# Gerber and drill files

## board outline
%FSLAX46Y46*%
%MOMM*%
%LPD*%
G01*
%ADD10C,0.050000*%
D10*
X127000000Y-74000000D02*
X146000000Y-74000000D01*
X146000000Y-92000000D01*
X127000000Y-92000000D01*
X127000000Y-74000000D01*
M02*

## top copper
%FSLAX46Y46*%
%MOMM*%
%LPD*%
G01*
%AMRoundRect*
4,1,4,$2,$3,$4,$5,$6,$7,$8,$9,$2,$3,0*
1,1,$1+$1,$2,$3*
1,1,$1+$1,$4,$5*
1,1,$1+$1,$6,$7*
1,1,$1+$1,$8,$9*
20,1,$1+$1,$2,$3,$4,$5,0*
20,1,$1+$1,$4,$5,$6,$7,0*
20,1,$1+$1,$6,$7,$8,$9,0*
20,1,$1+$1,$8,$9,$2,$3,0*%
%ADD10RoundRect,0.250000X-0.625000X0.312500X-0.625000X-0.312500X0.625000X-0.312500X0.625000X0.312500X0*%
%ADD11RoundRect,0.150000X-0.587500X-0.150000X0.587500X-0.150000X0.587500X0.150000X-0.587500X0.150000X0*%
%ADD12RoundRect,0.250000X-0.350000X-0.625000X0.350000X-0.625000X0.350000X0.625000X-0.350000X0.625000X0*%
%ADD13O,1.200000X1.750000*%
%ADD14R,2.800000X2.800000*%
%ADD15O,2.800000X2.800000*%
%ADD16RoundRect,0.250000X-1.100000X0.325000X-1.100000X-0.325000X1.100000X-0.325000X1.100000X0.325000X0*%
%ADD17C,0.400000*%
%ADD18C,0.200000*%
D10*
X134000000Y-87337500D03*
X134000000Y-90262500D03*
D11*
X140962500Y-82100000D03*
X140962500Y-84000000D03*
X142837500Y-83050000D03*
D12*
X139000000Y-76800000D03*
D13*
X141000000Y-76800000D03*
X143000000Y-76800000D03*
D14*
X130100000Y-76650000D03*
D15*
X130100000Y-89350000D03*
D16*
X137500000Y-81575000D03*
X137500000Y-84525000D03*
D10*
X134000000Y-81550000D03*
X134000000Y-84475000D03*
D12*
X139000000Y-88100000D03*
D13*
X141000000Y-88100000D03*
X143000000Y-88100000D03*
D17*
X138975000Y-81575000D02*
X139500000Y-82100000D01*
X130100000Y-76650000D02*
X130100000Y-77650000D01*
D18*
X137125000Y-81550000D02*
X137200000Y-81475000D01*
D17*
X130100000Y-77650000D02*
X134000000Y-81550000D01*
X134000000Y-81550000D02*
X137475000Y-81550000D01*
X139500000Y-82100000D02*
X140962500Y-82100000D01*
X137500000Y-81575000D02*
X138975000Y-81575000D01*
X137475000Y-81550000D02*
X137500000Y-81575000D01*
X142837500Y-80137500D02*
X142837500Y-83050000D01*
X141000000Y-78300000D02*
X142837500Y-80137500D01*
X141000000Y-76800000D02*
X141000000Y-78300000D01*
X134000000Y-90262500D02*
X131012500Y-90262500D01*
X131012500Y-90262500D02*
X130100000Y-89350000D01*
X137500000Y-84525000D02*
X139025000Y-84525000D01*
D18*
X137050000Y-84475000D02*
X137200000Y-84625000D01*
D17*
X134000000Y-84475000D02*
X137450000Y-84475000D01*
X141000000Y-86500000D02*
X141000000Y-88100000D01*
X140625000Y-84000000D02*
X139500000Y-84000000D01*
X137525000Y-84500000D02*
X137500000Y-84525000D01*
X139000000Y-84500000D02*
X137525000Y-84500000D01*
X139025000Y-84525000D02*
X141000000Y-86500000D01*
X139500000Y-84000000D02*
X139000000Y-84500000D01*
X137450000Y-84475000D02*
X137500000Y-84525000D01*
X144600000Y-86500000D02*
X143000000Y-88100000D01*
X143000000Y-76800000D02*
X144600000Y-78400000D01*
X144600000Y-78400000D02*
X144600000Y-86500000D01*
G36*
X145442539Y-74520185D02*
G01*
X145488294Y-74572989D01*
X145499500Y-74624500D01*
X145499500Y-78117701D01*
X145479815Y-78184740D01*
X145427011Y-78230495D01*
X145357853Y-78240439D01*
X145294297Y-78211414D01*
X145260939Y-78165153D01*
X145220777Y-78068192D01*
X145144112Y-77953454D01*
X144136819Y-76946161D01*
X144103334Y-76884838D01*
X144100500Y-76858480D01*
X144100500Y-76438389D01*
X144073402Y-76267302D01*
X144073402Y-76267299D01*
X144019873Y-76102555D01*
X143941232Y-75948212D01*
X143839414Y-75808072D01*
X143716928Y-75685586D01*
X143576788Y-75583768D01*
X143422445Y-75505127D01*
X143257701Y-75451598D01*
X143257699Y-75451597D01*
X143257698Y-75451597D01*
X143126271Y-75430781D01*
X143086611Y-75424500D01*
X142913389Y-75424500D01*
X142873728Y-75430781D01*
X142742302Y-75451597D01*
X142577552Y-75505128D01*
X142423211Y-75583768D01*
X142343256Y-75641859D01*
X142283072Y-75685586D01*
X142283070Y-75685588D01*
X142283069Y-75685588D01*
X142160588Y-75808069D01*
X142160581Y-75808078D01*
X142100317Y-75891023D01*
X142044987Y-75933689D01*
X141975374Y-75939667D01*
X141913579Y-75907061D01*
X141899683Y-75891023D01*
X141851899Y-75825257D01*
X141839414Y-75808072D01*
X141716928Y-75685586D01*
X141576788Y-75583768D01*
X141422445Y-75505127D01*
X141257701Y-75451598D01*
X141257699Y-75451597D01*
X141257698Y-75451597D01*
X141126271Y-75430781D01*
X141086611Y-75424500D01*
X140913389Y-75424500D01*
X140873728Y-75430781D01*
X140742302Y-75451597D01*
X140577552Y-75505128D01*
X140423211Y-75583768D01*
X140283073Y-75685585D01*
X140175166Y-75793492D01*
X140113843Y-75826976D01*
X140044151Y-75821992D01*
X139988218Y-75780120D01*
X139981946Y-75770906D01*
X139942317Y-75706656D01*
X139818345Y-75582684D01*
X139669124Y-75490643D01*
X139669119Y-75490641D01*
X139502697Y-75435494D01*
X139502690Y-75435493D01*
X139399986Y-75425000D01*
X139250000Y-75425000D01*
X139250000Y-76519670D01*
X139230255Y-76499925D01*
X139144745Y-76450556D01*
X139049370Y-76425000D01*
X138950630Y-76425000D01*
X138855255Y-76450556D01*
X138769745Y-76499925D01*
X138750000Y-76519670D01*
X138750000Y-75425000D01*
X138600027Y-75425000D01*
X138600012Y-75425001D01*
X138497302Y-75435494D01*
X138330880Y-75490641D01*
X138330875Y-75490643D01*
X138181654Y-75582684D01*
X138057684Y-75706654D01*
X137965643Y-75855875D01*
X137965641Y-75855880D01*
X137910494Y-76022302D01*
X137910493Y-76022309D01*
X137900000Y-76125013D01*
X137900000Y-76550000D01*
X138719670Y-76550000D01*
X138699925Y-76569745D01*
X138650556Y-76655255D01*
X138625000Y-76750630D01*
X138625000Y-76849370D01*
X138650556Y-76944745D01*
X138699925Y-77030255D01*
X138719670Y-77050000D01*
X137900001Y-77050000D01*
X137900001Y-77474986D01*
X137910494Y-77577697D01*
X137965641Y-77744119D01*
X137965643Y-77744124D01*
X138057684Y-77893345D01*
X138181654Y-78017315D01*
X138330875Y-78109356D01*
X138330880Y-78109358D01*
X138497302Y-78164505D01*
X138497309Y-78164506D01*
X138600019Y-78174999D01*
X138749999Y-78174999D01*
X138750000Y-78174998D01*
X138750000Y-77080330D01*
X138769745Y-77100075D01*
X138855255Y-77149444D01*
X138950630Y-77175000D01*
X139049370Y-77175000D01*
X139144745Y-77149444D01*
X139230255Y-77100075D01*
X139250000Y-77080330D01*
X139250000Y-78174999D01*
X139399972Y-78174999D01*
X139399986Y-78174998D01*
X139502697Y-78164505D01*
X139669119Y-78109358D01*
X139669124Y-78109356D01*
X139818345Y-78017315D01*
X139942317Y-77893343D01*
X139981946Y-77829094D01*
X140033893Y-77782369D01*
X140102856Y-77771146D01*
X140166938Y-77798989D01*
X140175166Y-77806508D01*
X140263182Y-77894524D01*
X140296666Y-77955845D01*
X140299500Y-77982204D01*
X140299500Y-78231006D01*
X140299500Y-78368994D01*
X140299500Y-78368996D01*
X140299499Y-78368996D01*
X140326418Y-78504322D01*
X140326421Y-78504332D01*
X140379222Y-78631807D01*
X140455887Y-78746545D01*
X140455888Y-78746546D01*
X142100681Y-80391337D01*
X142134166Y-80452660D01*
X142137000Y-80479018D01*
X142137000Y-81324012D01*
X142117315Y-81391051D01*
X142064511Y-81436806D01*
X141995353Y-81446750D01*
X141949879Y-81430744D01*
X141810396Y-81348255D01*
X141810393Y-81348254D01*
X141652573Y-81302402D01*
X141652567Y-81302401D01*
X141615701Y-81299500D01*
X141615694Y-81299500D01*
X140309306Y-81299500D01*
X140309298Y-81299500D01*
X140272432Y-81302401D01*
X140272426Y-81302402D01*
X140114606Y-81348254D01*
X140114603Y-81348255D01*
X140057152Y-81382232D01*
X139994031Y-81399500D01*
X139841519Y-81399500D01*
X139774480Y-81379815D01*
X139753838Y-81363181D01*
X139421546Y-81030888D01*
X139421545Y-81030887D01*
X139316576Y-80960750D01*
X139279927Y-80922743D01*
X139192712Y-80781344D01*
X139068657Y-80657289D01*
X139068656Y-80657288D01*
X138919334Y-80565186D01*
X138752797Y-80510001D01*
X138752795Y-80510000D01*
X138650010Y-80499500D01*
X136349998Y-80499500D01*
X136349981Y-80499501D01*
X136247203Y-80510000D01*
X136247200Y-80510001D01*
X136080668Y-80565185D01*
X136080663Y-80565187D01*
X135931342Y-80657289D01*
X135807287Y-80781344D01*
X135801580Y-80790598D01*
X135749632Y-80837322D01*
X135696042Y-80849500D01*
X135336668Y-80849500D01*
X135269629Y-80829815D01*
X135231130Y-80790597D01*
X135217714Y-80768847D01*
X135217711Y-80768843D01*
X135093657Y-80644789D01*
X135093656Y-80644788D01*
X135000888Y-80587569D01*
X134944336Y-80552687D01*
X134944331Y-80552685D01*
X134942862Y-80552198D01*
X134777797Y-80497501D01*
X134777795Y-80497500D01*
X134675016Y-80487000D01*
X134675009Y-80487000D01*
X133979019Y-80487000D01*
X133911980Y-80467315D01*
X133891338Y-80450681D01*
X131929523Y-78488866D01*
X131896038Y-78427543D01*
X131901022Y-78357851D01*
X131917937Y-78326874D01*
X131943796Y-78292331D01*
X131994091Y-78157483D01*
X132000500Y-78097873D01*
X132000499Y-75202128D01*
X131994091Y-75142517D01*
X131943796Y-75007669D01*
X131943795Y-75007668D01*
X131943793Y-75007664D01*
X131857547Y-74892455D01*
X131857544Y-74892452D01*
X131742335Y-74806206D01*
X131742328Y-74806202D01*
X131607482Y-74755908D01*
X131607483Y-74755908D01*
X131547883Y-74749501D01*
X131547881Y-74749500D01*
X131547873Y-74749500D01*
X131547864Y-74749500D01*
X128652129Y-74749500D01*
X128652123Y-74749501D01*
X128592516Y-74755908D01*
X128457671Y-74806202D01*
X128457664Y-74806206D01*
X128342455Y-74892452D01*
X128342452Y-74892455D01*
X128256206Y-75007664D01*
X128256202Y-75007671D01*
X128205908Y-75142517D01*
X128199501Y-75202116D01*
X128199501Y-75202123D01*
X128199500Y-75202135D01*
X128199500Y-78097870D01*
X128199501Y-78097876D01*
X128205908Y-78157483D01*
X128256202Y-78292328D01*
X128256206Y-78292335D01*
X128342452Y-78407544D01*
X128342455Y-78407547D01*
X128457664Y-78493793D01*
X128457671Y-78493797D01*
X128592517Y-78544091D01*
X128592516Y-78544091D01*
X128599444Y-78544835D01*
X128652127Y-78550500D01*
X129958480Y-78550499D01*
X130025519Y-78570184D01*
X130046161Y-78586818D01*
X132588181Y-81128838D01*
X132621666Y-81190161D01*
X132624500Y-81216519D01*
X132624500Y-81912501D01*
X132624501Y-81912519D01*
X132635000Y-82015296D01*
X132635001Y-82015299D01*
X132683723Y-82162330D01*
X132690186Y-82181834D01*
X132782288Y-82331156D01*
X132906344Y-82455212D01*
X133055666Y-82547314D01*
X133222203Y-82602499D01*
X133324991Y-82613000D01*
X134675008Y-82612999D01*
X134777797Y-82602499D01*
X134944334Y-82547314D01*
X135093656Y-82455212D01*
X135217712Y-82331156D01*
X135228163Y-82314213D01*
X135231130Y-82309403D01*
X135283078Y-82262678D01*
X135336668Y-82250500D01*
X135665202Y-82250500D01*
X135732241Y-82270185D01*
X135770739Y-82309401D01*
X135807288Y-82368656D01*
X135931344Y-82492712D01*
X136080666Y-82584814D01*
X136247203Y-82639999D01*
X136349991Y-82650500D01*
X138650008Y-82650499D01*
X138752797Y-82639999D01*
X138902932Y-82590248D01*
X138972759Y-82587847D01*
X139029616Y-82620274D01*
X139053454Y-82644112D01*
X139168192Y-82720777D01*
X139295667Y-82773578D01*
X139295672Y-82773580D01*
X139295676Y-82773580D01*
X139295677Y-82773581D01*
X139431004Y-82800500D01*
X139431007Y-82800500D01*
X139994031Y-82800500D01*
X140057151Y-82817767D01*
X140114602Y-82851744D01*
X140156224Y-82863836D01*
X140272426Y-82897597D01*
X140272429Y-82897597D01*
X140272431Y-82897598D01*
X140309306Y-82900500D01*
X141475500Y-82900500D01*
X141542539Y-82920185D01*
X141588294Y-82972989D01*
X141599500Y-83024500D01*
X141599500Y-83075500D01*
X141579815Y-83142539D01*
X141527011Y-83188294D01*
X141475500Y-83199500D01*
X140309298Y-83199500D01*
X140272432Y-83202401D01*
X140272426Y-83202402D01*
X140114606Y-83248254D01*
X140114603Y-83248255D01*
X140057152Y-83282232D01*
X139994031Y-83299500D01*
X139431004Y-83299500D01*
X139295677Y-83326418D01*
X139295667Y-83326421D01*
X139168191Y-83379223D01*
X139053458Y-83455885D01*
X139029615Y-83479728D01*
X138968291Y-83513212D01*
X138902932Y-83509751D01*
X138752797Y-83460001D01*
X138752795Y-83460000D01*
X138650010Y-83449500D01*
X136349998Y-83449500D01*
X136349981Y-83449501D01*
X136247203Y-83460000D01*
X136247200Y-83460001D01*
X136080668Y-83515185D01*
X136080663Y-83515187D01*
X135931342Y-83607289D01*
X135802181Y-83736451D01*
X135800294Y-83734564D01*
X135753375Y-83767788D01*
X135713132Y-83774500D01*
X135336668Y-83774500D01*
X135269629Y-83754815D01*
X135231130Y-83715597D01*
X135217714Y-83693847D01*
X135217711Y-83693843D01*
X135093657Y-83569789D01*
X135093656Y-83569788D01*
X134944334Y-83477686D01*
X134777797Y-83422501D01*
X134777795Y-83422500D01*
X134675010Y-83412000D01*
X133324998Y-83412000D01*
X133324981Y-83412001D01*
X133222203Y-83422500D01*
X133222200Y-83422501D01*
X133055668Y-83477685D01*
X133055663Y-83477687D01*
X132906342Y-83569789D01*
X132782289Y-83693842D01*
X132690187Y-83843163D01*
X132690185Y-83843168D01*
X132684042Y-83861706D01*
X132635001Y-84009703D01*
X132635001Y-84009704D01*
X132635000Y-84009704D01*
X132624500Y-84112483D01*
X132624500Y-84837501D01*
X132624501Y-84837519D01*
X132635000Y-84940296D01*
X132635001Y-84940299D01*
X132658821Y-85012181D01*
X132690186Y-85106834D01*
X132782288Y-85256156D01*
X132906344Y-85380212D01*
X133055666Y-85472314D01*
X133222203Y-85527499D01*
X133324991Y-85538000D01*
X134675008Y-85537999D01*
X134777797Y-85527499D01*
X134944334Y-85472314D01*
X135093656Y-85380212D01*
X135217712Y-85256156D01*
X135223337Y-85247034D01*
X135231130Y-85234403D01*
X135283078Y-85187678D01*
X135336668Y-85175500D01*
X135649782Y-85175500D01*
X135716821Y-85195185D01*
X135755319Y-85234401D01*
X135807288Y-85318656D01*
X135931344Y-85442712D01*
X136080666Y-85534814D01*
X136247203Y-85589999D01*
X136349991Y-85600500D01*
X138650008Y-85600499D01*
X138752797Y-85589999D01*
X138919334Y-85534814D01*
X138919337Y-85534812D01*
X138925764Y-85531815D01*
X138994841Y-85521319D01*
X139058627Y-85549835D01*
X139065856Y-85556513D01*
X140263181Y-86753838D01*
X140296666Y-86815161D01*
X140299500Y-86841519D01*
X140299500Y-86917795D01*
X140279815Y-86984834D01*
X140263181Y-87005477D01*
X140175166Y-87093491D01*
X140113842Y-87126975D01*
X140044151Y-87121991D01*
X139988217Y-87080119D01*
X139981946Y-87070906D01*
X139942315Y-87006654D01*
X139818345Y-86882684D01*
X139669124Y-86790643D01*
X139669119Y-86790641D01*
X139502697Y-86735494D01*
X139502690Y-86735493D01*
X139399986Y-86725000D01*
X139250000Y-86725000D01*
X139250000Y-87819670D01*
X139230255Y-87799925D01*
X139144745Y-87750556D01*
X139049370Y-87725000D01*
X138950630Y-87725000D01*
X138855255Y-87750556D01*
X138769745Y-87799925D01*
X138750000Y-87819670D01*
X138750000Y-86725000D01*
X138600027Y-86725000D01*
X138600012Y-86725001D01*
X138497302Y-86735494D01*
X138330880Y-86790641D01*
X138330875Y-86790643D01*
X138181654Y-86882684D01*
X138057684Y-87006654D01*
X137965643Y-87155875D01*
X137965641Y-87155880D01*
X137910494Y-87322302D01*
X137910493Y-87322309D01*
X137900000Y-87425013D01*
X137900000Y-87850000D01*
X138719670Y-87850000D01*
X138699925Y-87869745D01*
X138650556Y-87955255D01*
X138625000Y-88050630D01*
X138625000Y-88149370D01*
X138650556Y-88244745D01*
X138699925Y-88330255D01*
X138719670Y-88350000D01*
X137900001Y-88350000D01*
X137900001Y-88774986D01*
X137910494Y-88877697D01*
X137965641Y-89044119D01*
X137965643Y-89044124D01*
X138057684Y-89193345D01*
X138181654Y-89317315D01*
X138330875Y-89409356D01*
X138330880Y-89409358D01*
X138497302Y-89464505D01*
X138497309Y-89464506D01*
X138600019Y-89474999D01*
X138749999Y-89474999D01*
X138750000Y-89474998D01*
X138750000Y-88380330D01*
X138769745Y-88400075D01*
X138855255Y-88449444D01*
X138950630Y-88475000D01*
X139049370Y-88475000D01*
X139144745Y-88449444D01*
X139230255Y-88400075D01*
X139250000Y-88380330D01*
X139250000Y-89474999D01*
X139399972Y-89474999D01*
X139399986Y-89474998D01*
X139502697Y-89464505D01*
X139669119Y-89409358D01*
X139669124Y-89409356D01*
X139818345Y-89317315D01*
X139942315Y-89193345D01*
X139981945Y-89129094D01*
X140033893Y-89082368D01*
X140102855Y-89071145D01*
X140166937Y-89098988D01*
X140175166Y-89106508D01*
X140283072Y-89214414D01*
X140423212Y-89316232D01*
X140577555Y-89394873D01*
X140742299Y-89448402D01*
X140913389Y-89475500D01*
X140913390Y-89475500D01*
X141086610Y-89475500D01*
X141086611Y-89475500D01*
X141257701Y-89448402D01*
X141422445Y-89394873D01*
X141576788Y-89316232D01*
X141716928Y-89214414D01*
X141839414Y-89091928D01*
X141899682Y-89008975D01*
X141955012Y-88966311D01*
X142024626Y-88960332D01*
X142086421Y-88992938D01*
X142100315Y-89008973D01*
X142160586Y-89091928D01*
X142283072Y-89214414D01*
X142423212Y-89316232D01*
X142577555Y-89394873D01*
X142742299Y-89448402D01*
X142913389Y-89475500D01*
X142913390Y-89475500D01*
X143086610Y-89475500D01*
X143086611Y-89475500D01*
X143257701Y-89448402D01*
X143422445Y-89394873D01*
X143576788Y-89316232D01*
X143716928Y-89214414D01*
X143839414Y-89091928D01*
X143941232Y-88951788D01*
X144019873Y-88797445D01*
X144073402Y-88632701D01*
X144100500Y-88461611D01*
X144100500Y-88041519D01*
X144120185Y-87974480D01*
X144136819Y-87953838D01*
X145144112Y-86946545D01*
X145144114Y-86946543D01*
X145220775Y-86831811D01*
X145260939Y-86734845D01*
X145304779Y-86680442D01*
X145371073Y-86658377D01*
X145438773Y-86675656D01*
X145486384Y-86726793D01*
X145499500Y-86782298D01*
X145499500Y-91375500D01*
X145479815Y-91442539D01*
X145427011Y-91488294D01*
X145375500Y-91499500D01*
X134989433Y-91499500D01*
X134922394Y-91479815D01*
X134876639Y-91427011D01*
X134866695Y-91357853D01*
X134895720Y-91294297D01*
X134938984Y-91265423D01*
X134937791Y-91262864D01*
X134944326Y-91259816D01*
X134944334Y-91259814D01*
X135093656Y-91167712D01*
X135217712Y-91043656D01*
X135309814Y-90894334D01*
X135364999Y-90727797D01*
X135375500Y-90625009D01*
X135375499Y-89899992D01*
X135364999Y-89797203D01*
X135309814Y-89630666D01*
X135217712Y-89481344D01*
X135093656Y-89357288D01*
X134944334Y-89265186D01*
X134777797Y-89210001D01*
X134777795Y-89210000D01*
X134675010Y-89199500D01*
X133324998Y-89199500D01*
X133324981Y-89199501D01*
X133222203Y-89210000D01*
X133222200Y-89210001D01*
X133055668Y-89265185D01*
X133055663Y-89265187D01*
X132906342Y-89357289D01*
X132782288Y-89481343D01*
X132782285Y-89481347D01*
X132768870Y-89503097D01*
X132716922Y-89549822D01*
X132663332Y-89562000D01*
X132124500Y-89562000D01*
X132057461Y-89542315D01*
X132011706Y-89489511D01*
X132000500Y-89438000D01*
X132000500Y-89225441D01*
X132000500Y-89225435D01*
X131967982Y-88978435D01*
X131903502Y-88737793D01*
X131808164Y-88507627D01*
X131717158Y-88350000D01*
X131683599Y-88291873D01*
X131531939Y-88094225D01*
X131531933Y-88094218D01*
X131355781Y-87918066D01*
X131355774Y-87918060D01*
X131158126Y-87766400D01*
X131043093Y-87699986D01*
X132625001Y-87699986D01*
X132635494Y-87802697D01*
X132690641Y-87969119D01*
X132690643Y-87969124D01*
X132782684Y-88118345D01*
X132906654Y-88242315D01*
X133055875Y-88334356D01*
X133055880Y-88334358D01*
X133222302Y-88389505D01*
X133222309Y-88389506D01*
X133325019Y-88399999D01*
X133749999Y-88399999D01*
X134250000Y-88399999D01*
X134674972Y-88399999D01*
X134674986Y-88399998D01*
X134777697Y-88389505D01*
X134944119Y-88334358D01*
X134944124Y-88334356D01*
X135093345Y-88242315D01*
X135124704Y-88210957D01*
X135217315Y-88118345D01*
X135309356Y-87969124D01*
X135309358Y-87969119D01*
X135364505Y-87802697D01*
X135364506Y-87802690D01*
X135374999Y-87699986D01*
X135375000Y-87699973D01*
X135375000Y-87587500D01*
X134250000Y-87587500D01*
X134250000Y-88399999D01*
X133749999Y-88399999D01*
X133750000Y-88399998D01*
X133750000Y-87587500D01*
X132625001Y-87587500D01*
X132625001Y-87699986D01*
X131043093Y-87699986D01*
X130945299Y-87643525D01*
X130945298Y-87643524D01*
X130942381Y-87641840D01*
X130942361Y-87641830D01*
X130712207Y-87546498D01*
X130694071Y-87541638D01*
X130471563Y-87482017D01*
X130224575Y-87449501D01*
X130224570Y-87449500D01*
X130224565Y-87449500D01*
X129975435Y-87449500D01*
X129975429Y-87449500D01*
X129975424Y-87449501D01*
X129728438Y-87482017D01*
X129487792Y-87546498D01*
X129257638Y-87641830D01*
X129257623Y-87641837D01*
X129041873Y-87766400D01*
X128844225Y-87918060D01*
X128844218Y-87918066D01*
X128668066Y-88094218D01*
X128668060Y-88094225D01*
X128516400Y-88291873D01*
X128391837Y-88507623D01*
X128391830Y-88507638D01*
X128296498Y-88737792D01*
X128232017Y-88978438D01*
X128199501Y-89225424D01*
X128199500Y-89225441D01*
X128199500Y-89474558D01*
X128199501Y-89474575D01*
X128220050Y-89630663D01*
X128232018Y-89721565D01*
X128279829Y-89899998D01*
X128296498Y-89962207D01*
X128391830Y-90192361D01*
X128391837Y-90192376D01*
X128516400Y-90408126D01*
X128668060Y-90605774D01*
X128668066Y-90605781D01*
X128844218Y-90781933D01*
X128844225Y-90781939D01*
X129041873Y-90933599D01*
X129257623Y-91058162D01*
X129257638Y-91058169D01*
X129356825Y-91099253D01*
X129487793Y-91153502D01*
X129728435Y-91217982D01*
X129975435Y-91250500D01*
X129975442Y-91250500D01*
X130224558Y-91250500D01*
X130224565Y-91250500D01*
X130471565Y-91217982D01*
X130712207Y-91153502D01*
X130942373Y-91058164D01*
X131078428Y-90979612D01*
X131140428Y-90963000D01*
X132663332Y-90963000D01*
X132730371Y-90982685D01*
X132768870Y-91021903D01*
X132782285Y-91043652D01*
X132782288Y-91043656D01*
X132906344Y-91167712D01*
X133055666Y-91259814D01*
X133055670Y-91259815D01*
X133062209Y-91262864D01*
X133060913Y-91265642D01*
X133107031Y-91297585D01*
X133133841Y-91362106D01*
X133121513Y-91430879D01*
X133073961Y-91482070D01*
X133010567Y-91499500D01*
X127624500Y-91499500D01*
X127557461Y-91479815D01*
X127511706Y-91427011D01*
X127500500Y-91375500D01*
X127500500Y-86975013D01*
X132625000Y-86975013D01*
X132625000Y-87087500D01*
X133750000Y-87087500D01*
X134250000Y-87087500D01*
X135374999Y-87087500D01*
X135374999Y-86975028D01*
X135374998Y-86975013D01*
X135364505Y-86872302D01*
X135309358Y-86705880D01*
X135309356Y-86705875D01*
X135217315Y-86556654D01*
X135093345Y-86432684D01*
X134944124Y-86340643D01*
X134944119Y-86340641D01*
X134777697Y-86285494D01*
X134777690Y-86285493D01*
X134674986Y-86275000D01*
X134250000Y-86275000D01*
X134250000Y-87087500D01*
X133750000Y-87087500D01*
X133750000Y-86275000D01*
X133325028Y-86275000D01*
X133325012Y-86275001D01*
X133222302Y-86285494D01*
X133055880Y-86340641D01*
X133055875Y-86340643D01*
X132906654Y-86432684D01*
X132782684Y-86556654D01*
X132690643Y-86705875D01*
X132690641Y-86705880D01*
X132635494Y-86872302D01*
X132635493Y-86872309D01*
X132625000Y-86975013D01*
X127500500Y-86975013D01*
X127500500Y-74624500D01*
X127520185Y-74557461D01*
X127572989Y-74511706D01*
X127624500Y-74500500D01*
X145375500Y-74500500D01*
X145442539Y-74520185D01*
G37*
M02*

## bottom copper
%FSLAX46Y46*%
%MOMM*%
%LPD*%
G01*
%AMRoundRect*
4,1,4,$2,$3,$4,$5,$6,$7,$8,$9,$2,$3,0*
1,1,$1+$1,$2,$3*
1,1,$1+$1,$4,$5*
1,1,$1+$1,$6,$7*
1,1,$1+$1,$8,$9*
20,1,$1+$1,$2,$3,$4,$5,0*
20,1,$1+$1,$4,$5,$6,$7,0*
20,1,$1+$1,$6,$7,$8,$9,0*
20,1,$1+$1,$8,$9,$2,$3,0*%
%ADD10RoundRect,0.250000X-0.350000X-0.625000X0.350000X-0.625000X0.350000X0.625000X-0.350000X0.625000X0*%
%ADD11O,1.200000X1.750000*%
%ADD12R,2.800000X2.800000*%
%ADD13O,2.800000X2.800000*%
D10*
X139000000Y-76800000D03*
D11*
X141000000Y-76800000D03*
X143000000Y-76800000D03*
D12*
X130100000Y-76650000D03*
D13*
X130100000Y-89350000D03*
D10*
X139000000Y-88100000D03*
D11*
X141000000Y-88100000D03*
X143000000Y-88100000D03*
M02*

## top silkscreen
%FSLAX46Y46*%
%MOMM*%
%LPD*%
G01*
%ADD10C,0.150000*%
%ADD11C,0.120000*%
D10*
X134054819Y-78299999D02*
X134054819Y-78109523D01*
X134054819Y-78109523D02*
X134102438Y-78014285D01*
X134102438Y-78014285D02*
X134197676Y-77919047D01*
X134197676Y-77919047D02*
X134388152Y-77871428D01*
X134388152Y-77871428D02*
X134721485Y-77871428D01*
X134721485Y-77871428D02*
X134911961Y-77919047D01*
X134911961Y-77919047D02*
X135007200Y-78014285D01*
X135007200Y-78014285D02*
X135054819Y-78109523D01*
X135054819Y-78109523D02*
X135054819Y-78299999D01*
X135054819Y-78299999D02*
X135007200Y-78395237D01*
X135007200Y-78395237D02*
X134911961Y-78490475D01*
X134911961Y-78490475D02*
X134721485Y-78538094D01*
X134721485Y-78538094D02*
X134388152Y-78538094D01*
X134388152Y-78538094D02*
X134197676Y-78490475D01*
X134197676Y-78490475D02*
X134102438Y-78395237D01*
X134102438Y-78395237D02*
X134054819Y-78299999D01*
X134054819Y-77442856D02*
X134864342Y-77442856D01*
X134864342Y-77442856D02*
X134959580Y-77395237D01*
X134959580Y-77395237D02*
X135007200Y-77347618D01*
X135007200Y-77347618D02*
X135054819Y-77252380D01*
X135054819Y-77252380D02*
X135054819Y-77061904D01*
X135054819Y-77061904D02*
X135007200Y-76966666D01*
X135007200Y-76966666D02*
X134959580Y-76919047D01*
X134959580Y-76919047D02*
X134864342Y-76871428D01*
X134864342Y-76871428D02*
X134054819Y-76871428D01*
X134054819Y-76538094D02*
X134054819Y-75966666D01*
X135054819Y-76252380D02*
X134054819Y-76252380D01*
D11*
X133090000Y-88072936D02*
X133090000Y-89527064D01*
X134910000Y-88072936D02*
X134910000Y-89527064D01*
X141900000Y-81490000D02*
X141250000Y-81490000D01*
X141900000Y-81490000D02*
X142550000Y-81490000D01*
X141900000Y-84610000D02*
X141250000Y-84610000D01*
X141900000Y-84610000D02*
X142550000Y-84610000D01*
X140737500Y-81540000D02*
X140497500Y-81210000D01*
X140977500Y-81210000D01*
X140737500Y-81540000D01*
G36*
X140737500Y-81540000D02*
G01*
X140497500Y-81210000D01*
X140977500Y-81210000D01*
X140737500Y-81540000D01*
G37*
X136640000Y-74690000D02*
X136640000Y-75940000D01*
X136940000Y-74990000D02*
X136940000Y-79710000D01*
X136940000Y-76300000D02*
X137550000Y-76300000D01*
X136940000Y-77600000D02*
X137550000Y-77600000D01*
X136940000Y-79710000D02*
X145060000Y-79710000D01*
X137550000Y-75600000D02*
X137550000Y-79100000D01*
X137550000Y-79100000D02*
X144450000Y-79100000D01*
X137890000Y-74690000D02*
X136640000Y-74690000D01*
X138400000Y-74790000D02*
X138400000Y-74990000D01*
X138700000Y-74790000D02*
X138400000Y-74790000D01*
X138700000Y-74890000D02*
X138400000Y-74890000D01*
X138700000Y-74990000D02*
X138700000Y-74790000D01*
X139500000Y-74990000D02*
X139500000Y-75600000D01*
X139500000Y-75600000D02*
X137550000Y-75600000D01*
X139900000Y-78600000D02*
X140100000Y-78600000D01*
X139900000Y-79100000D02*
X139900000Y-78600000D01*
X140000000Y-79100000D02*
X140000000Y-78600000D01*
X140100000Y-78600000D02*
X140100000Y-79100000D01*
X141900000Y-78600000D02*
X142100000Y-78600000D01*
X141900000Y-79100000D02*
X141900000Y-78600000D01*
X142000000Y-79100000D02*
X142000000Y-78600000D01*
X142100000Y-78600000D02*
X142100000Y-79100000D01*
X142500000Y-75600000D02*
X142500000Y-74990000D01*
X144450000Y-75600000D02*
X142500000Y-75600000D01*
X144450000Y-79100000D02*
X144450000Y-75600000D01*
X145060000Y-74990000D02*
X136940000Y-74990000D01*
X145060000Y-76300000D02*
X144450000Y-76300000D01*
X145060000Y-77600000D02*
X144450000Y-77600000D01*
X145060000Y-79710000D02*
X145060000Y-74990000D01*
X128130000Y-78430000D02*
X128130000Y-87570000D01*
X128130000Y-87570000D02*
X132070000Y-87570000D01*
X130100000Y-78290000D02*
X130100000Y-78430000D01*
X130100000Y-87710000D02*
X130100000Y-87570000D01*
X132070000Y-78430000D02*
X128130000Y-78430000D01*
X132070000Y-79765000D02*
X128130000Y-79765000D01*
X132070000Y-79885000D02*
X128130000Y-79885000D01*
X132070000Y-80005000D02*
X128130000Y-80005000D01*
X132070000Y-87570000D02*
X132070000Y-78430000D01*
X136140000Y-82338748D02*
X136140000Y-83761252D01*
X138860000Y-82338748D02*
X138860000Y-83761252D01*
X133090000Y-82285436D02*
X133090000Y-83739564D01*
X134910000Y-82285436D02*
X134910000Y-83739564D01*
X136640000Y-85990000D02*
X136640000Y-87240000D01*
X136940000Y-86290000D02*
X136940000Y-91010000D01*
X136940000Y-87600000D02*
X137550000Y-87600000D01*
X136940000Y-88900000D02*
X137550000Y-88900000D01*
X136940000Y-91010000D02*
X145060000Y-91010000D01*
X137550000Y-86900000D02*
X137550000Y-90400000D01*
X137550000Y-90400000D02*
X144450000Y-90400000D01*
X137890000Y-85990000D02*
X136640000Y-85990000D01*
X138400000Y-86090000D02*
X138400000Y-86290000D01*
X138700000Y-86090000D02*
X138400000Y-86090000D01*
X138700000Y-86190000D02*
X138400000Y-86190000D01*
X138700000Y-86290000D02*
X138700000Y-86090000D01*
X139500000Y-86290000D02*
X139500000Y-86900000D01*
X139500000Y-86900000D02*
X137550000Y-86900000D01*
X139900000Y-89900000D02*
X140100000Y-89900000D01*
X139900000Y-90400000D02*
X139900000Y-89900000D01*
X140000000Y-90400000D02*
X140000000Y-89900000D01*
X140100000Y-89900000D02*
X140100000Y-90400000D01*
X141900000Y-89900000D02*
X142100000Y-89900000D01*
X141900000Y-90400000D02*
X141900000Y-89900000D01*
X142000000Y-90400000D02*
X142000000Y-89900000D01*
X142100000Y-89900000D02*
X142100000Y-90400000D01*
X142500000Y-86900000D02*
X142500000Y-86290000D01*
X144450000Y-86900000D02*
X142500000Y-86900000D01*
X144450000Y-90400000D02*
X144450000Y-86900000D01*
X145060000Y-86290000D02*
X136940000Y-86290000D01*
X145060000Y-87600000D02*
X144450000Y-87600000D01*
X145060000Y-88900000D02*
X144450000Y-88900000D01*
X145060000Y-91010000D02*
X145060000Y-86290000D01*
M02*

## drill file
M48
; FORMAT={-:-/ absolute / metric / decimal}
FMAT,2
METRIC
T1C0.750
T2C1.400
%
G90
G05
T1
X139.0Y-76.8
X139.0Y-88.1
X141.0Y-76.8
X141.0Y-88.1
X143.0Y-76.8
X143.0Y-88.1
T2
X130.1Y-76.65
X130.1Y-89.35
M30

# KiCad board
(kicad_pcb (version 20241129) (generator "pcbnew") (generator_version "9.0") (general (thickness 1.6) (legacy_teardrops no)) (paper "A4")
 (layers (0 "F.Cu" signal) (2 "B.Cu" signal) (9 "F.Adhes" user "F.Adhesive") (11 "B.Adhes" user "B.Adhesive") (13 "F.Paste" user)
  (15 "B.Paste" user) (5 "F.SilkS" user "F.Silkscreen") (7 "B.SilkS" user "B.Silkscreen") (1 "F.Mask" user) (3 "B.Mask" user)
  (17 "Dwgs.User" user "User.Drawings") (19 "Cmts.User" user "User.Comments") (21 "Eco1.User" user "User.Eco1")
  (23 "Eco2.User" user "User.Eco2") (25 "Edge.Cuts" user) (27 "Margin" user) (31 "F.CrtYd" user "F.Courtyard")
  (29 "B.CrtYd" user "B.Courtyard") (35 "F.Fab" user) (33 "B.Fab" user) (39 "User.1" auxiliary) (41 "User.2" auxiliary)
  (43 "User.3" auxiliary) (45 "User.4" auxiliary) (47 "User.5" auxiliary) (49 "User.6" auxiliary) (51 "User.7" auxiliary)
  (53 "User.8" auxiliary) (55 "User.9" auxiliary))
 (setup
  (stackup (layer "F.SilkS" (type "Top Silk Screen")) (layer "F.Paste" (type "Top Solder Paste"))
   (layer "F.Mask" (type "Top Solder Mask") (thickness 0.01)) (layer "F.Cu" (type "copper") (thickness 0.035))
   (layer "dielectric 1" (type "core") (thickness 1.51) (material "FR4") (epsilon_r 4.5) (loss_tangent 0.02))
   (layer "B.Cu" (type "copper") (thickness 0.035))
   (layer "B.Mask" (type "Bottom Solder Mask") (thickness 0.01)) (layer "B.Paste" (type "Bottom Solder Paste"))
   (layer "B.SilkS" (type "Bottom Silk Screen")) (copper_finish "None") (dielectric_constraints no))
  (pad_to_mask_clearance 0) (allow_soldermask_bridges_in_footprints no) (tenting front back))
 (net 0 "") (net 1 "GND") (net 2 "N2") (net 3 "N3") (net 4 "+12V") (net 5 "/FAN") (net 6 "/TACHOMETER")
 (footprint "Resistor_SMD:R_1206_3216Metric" (layer "F.Cu") (at 134 88.8 -90)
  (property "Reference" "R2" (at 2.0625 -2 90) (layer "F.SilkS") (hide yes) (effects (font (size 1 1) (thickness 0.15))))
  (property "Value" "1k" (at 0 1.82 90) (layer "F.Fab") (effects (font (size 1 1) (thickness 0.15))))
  (fp_line (start -0.727064 0.91) (end 0.727064 0.91) (stroke (width 0.12) (type solid)) (layer "F.SilkS"))
  (fp_line (start -0.727064 -0.91) (end 0.727064 -0.91) (stroke (width 0.12) (type solid)) (layer "F.SilkS"))
  (pad "1" smd roundrect (at -1.4625 0 270) (size 1.125 1.75) (layers "F.Cu" "F.Mask" "F.Paste") (roundrect_rratio 0.222222) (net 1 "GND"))
  (pad "2" smd roundrect (at 1.4625 0 270) (size 1.125 1.75) (layers "F.Cu" "F.Mask" "F.Paste") (roundrect_rratio 0.222222) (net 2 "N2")))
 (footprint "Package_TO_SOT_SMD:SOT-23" (layer "F.Cu") (at 141.9 83.05)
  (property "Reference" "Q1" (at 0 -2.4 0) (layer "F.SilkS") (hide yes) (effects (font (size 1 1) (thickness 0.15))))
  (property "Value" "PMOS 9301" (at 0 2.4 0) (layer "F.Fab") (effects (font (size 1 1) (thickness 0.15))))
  (fp_line (start 0 -1.56) (end -0.65 -1.56) (stroke (width 0.12) (type solid)) (layer "F.SilkS"))
  (fp_line (start 0 -1.56) (end 0.65 -1.56) (stroke (width 0.12) (type solid)) (layer "F.SilkS"))
  (fp_line (start 0 1.56) (end -0.65 1.56) (stroke (width 0.12) (type solid)) (layer "F.SilkS"))
  (fp_line (start 0 1.56) (end 0.65 1.56) (stroke (width 0.12) (type solid)) (layer "F.SilkS"))
  (fp_poly
   (pts (xy -1.1625 -1.51) (xy -1.4025 -1.84) (xy -0.9225 -1.84) (xy -1.1625 -1.51)) (stroke (width 0.12) (type solid)) (fill yes)
   (layer "F.SilkS"))
  (pad "1" smd roundrect (at -0.9375 -0.95) (size 1.475 0.6) (layers "F.Cu" "F.Mask" "F.Paste") (roundrect_rratio 0.25) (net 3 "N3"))
  (pad "2" smd roundrect (at -0.9375 0.95) (size 1.475 0.6) (layers "F.Cu" "F.Mask" "F.Paste") (roundrect_rratio 0.25) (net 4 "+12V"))
  (pad "3" smd roundrect (at 0.9375 0) (size 1.475 0.6) (layers "F.Cu" "F.Mask" "F.Paste") (roundrect_rratio 0.25) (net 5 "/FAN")))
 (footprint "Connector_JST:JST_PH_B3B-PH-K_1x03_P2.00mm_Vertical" (layer "F.Cu") (at 139 76.8)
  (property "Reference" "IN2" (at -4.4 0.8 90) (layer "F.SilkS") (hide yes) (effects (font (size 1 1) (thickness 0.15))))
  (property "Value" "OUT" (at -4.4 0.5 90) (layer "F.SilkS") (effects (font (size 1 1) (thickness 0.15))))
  (fp_line (start -2.36 -2.11) (end -2.36 -0.86) (stroke (width 0.12) (type solid)) (layer "F.SilkS"))
  (fp_line (start -2.06 -1.81) (end -2.06 2.91) (stroke (width 0.12) (type solid)) (layer "F.SilkS"))
  (fp_line (start -2.06 -0.5) (end -1.45 -0.5) (stroke (width 0.12) (type solid)) (layer "F.SilkS"))
  (fp_line (start -2.06 0.8) (end -1.45 0.8) (stroke (width 0.12) (type solid)) (layer "F.SilkS"))
  (fp_line (start -2.06 2.91) (end 6.06 2.91) (stroke (width 0.12) (type solid)) (layer "F.SilkS"))
  (fp_line (start -1.45 -1.2) (end -1.45 2.3) (stroke (width 0.12) (type solid)) (layer "F.SilkS"))
  (fp_line (start -1.45 2.3) (end 5.45 2.3) (stroke (width 0.12) (type solid)) (layer "F.SilkS"))
  (fp_line (start -1.11 -2.11) (end -2.36 -2.11) (stroke (width 0.12) (type solid)) (layer "F.SilkS"))
  (fp_line (start -0.6 -2.01) (end -0.6 -1.81) (stroke (width 0.12) (type solid)) (layer "F.SilkS"))
  (fp_line (start -0.3 -2.01) (end -0.6 -2.01) (stroke (width 0.12) (type solid)) (layer "F.SilkS"))
  (fp_line (start -0.3 -1.91) (end -0.6 -1.91) (stroke (width 0.12) (type solid)) (layer "F.SilkS"))
  (fp_line (start -0.3 -1.81) (end -0.3 -2.01) (stroke (width 0.12) (type solid)) (layer "F.SilkS"))
  (fp_line (start 0.5 -1.81) (end 0.5 -1.2) (stroke (width 0.12) (type solid)) (layer "F.SilkS"))
  (fp_line (start 0.5 -1.2) (end -1.45 -1.2) (stroke (width 0.12) (type solid)) (layer "F.SilkS"))
  (fp_line (start 0.9 1.8) (end 1.1 1.8) (stroke (width 0.12) (type solid)) (layer "F.SilkS"))
  (fp_line (start 0.9 2.3) (end 0.9 1.8) (stroke (width 0.12) (type solid)) (layer "F.SilkS"))
  (fp_line (start 1 2.3) (end 1 1.8) (stroke (width 0.12) (type solid)) (layer "F.SilkS"))
  (fp_line (start 1.1 1.8) (end 1.1 2.3) (stroke (width 0.12) (type solid)) (layer "F.SilkS"))
  (fp_line (start 2.9 1.8) (end 3.1 1.8) (stroke (width 0.12) (type solid)) (layer "F.SilkS"))
  (fp_line (start 2.9 2.3) (end 2.9 1.8) (stroke (width 0.12) (type solid)) (layer "F.SilkS"))
  (fp_line (start 3 2.3) (end 3 1.8) (stroke (width 0.12) (type solid)) (layer "F.SilkS"))
  (fp_line (start 3.1 1.8) (end 3.1 2.3) (stroke (width 0.12) (type solid)) (layer "F.SilkS"))
  (fp_line (start 3.5 -1.2) (end 3.5 -1.81) (stroke (width 0.12) (type solid)) (layer "F.SilkS"))
  (fp_line (start 5.45 -1.2) (end 3.5 -1.2) (stroke (width 0.12) (type solid)) (layer "F.SilkS"))
  (fp_line (start 5.45 2.3) (end 5.45 -1.2) (stroke (width 0.12) (type solid)) (layer "F.SilkS"))
  (fp_line (start 6.06 -1.81) (end -2.06 -1.81) (stroke (width 0.12) (type solid)) (layer "F.SilkS"))
  (fp_line (start 6.06 -0.5) (end 5.45 -0.5) (stroke (width 0.12) (type solid)) (layer "F.SilkS"))
  (fp_line (start 6.06 0.8) (end 5.45 0.8) (stroke (width 0.12) (type solid)) (layer "F.SilkS"))
  (fp_line (start 6.06 2.91) (end 6.06 -1.81) (stroke (width 0.12) (type solid)) (layer "F.SilkS"))
  (pad "1" thru_hole roundrect (at 0 0) (size 1.2 1.75) (drill 0.75) (layers "*.Cu" "*.Mask") (remove_unused_layers no)
   (roundrect_rratio 0.208333) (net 1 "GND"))
  (pad "2" thru_hole oval (at 2 0) (size 1.2 1.75) (drill 0.75) (layers "*.Cu" "*.Mask") (remove_unused_layers no) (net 5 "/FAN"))
  (pad "3" thru_hole oval (at 4 0) (size 1.2 1.75) (drill 0.75) (layers "*.Cu" "*.Mask") (remove_unused_layers no) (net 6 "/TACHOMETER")))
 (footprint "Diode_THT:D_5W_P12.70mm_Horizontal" (layer "F.Cu") (at 130.1 76.65 -90)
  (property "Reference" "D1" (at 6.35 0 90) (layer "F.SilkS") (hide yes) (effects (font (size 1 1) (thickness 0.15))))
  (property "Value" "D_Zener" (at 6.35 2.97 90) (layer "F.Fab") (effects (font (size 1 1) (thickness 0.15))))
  (fp_line (start 1.78 1.97) (end 10.92 1.97) (stroke (width 0.12) (type solid)) (layer "F.SilkS"))
  (fp_line (start 10.92 1.97) (end 10.92 -1.97) (stroke (width 0.12) (type solid)) (layer "F.SilkS"))
  (fp_line (start 1.64 0) (end 1.78 0) (stroke (width 0.12) (type solid)) (layer "F.SilkS"))
  (fp_line (start 11.06 0) (end 10.92 0) (stroke (width 0.12) (type solid)) (layer "F.SilkS"))
  (fp_line (start 1.78 -1.97) (end 1.78 1.97) (stroke (width 0.12) (type solid)) (layer "F.SilkS"))
  (fp_line (start 3.115 -1.97) (end 3.115 1.97) (stroke (width 0.12) (type solid)) (layer "F.SilkS"))
  (fp_line (start 3.235 -1.97) (end 3.235 1.97) (stroke (width 0.12) (type solid)) (layer "F.SilkS"))
  (fp_line (start 3.355 -1.97) (end 3.355 1.97) (stroke (width 0.12) (type solid)) (layer "F.SilkS"))
  (fp_line (start 10.92 -1.97) (end 1.78 -1.97) (stroke (width 0.12) (type solid)) (layer "F.SilkS"))
  (pad "1" thru_hole rect (at 0 0 270) (size 2.8 2.8) (drill 1.4) (layers "*.Cu" "*.Mask") (remove_unused_layers no) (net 3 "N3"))
  (pad "2" thru_hole oval (at 12.7 0 270) (size 2.8 2.8) (drill 1.4) (layers "*.Cu" "*.Mask") (remove_unused_layers no) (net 2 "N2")))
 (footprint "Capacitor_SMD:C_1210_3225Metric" (layer "F.Cu") (at 137.5 83.05 -90)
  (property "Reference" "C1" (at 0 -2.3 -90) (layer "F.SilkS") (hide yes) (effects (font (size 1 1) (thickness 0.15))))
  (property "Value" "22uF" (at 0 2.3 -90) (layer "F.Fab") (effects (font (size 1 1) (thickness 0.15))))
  (fp_line (start -0.711252 1.36) (end 0.711252 1.36) (stroke (width 0.12) (type solid)) (layer "F.SilkS"))
  (fp_line (start -0.711252 -1.36) (end 0.711252 -1.36) (stroke (width 0.12) (type solid)) (layer "F.SilkS"))
  (pad "1" smd roundrect (at -1.475 0 270) (size 1.15 2.7) (layers "F.Cu" "F.Mask" "F.Paste") (roundrect_rratio 0.217391) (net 3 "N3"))
  (pad "2" smd roundrect (at 1.475 0 270) (size 1.15 2.7) (layers "F.Cu" "F.Mask" "F.Paste") (roundrect_rratio 0.217391) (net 4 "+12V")))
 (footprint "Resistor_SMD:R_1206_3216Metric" (layer "F.Cu") (at 134 83.0125 -90)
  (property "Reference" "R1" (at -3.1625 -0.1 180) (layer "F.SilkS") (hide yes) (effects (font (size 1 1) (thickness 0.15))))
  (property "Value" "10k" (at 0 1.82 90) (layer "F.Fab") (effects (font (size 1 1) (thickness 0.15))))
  (fp_line (start -0.727064 0.91) (end 0.727064 0.91) (stroke (width 0.12) (type solid)) (layer "F.SilkS"))
  (fp_line (start -0.727064 -0.91) (end 0.727064 -0.91) (stroke (width 0.12) (type solid)) (layer "F.SilkS"))
  (pad "1" smd roundrect (at -1.4625 0 270) (size 1.125 1.75) (layers "F.Cu" "F.Mask" "F.Paste") (roundrect_rratio 0.222222) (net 3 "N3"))
  (pad "2" smd roundrect (at 1.4625 0 270) (size 1.125 1.75) (layers "F.Cu" "F.Mask" "F.Paste") (roundrect_rratio 0.222222) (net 4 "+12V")))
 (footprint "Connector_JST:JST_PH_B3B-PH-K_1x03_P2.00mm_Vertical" (layer "F.Cu") (at 139 88.1)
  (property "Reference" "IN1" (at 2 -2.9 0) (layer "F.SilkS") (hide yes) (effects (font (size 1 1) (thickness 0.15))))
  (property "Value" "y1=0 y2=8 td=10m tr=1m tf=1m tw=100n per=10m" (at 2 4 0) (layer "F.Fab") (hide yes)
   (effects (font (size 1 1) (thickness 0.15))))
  (fp_line (start -2.36 -2.11) (end -2.36 -0.86) (stroke (width 0.12) (type solid)) (layer "F.SilkS"))
  (fp_line (start -2.06 -1.81) (end -2.06 2.91) (stroke (width 0.12) (type solid)) (layer "F.SilkS"))
  (fp_line (start -2.06 -0.5) (end -1.45 -0.5) (stroke (width 0.12) (type solid)) (layer "F.SilkS"))
  (fp_line (start -2.06 0.8) (end -1.45 0.8) (stroke (width 0.12) (type solid)) (layer "F.SilkS"))
  (fp_line (start -2.06 2.91) (end 6.06 2.91) (stroke (width 0.12) (type solid)) (layer "F.SilkS"))
  (fp_line (start -1.45 -1.2) (end -1.45 2.3) (stroke (width 0.12) (type solid)) (layer "F.SilkS"))
  (fp_line (start -1.45 2.3) (end 5.45 2.3) (stroke (width 0.12) (type solid)) (layer "F.SilkS"))
  (fp_line (start -1.11 -2.11) (end -2.36 -2.11) (stroke (width 0.12) (type solid)) (layer "F.SilkS"))
  (fp_line (start -0.6 -2.01) (end -0.6 -1.81) (stroke (width 0.12) (type solid)) (layer "F.SilkS"))
  (fp_line (start -0.3 -2.01) (end -0.6 -2.01) (stroke (width 0.12) (type solid)) (layer "F.SilkS"))
  (fp_line (start -0.3 -1.91) (end -0.6 -1.91) (stroke (width 0.12) (type solid)) (layer "F.SilkS"))
  (fp_line (start -0.3 -1.81) (end -0.3 -2.01) (stroke (width 0.12) (type solid)) (layer "F.SilkS"))
  (fp_line (start 0.5 -1.81) (end 0.5 -1.2) (stroke (width 0.12) (type solid)) (layer "F.SilkS"))
  (fp_line (start 0.5 -1.2) (end -1.45 -1.2) (stroke (width 0.12) (type solid)) (layer "F.SilkS"))
  (fp_line (start 0.9 1.8) (end 1.1 1.8) (stroke (width 0.12) (type solid)) (layer "F.SilkS"))
  (fp_line (start 0.9 2.3) (end 0.9 1.8) (stroke (width 0.12) (type solid)) (layer "F.SilkS"))
  (fp_line (start 1 2.3) (end 1 1.8) (stroke (width 0.12) (type solid)) (layer "F.SilkS"))
  (fp_line (start 1.1 1.8) (end 1.1 2.3) (stroke (width 0.12) (type solid)) (layer "F.SilkS"))
  (fp_line (start 2.9 1.8) (end 3.1 1.8) (stroke (width 0.12) (type solid)) (layer "F.SilkS"))
  (fp_line (start 2.9 2.3) (end 2.9 1.8) (stroke (width 0.12) (type solid)) (layer "F.SilkS"))
  (fp_line (start 3 2.3) (end 3 1.8) (stroke (width 0.12) (type solid)) (layer "F.SilkS"))
  (fp_line (start 3.1 1.8) (end 3.1 2.3) (stroke (width 0.12) (type solid)) (layer "F.SilkS"))
  (fp_line (start 3.5 -1.2) (end 3.5 -1.81) (stroke (width 0.12) (type solid)) (layer "F.SilkS"))
  (fp_line (start 5.45 -1.2) (end 3.5 -1.2) (stroke (width 0.12) (type solid)) (layer "F.SilkS"))
  (fp_line (start 5.45 2.3) (end 5.45 -1.2) (stroke (width 0.12) (type solid)) (layer "F.SilkS"))
  (fp_line (start 6.06 -1.81) (end -2.06 -1.81) (stroke (width 0.12) (type solid)) (layer "F.SilkS"))
  (fp_line (start 6.06 -0.5) (end 5.45 -0.5) (stroke (width 0.12) (type solid)) (layer "F.SilkS"))
  (fp_line (start 6.06 0.8) (end 5.45 0.8) (stroke (width 0.12) (type solid)) (layer "F.SilkS"))
  (fp_line (start 6.06 2.91) (end 6.06 -1.81) (stroke (width 0.12) (type solid)) (layer "F.SilkS"))
  (pad "1" thru_hole roundrect (at 0 0) (size 1.2 1.75) (drill 0.75) (layers "*.Cu" "*.Mask") (remove_unused_layers no)
   (roundrect_rratio 0.208333) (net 1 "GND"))
  (pad "2" thru_hole oval (at 2 0) (size 1.2 1.75) (drill 0.75) (layers "*.Cu" "*.Mask") (remove_unused_layers no) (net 4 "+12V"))
  (pad "3" thru_hole oval (at 4 0) (size 1.2 1.75) (drill 0.75) (layers "*.Cu" "*.Mask") (remove_unused_layers no) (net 6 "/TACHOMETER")))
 (gr_rect (start 127 74) (end 146 92) (stroke (width 0.05) (type default)) (fill no) (layer "Edge.Cuts"))
 (segment (start 138.975 81.575) (end 139.5 82.1) (width 0.4) (layer "F.Cu") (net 3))
 (segment (start 130.1 76.65) (end 130.1 77.65) (width 0.4) (layer "F.Cu") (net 3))
 (segment (start 137.125 81.55) (end 137.2 81.475) (width 0.2) (layer "F.Cu") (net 3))
 (segment (start 130.1 77.65) (end 134 81.55) (width 0.4) (layer "F.Cu") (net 3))
 (segment (start 134 81.55) (end 137.475 81.55) (width 0.4) (layer "F.Cu") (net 3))
 (segment (start 139.5 82.1) (end 140.9625 82.1) (width 0.4) (layer "F.Cu") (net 3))
 (segment (start 137.5 81.575) (end 138.975 81.575) (width 0.4) (layer "F.Cu") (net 3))
 (segment (start 137.475 81.55) (end 137.5 81.575) (width 0.4) (layer "F.Cu") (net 3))
 (segment (start 142.8375 80.1375) (end 142.8375 83.05) (width 0.4) (layer "F.Cu") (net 5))
 (segment (start 141 78.3) (end 142.8375 80.1375) (width 0.4) (layer "F.Cu") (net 5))
 (segment (start 141 76.8) (end 141 78.3) (width 0.4) (layer "F.Cu") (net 5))
 (segment (start 134 90.2625) (end 131.0125 90.2625) (width 0.4) (layer "F.Cu") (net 2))
 (segment (start 131.0125 90.2625) (end 130.1 89.35) (width 0.4) (layer "F.Cu") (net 2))
 (segment (start 137.5 84.525) (end 139.025 84.525) (width 0.4) (layer "F.Cu") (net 4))
 (segment (start 137.05 84.475) (end 137.2 84.625) (width 0.2) (layer "F.Cu") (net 4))
 (segment (start 134 84.475) (end 137.45 84.475) (width 0.4) (layer "F.Cu") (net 4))
 (segment (start 141 86.5) (end 141 88.1) (width 0.4) (layer "F.Cu") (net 4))
 (segment (start 140.625 84) (end 139.5 84) (width 0.4) (layer "F.Cu") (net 4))
 (segment (start 137.525 84.5) (end 137.5 84.525) (width 0.4) (layer "F.Cu") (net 4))
 (segment (start 139 84.5) (end 137.525 84.5) (width 0.4) (layer "F.Cu") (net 4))
 (segment (start 139.025 84.525) (end 141 86.5) (width 0.4) (layer "F.Cu") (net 4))
 (segment (start 139.5 84) (end 139 84.5) (width 0.4) (layer "F.Cu") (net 4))
 (segment (start 137.45 84.475) (end 137.5 84.525) (width 0.4) (layer "F.Cu") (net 4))
 (segment (start 144.6 86.5) (end 143 88.1) (width 0.4) (layer "F.Cu") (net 6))
 (segment (start 143 76.8) (end 144.6 78.4) (width 0.4) (layer "F.Cu") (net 6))
 (segment (start 144.6 78.4) (end 144.6 86.5) (width 0.4) (layer "F.Cu") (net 6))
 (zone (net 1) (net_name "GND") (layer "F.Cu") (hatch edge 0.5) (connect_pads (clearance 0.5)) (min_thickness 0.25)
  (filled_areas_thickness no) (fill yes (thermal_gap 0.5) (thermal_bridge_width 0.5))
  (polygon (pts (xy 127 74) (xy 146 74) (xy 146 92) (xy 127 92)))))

